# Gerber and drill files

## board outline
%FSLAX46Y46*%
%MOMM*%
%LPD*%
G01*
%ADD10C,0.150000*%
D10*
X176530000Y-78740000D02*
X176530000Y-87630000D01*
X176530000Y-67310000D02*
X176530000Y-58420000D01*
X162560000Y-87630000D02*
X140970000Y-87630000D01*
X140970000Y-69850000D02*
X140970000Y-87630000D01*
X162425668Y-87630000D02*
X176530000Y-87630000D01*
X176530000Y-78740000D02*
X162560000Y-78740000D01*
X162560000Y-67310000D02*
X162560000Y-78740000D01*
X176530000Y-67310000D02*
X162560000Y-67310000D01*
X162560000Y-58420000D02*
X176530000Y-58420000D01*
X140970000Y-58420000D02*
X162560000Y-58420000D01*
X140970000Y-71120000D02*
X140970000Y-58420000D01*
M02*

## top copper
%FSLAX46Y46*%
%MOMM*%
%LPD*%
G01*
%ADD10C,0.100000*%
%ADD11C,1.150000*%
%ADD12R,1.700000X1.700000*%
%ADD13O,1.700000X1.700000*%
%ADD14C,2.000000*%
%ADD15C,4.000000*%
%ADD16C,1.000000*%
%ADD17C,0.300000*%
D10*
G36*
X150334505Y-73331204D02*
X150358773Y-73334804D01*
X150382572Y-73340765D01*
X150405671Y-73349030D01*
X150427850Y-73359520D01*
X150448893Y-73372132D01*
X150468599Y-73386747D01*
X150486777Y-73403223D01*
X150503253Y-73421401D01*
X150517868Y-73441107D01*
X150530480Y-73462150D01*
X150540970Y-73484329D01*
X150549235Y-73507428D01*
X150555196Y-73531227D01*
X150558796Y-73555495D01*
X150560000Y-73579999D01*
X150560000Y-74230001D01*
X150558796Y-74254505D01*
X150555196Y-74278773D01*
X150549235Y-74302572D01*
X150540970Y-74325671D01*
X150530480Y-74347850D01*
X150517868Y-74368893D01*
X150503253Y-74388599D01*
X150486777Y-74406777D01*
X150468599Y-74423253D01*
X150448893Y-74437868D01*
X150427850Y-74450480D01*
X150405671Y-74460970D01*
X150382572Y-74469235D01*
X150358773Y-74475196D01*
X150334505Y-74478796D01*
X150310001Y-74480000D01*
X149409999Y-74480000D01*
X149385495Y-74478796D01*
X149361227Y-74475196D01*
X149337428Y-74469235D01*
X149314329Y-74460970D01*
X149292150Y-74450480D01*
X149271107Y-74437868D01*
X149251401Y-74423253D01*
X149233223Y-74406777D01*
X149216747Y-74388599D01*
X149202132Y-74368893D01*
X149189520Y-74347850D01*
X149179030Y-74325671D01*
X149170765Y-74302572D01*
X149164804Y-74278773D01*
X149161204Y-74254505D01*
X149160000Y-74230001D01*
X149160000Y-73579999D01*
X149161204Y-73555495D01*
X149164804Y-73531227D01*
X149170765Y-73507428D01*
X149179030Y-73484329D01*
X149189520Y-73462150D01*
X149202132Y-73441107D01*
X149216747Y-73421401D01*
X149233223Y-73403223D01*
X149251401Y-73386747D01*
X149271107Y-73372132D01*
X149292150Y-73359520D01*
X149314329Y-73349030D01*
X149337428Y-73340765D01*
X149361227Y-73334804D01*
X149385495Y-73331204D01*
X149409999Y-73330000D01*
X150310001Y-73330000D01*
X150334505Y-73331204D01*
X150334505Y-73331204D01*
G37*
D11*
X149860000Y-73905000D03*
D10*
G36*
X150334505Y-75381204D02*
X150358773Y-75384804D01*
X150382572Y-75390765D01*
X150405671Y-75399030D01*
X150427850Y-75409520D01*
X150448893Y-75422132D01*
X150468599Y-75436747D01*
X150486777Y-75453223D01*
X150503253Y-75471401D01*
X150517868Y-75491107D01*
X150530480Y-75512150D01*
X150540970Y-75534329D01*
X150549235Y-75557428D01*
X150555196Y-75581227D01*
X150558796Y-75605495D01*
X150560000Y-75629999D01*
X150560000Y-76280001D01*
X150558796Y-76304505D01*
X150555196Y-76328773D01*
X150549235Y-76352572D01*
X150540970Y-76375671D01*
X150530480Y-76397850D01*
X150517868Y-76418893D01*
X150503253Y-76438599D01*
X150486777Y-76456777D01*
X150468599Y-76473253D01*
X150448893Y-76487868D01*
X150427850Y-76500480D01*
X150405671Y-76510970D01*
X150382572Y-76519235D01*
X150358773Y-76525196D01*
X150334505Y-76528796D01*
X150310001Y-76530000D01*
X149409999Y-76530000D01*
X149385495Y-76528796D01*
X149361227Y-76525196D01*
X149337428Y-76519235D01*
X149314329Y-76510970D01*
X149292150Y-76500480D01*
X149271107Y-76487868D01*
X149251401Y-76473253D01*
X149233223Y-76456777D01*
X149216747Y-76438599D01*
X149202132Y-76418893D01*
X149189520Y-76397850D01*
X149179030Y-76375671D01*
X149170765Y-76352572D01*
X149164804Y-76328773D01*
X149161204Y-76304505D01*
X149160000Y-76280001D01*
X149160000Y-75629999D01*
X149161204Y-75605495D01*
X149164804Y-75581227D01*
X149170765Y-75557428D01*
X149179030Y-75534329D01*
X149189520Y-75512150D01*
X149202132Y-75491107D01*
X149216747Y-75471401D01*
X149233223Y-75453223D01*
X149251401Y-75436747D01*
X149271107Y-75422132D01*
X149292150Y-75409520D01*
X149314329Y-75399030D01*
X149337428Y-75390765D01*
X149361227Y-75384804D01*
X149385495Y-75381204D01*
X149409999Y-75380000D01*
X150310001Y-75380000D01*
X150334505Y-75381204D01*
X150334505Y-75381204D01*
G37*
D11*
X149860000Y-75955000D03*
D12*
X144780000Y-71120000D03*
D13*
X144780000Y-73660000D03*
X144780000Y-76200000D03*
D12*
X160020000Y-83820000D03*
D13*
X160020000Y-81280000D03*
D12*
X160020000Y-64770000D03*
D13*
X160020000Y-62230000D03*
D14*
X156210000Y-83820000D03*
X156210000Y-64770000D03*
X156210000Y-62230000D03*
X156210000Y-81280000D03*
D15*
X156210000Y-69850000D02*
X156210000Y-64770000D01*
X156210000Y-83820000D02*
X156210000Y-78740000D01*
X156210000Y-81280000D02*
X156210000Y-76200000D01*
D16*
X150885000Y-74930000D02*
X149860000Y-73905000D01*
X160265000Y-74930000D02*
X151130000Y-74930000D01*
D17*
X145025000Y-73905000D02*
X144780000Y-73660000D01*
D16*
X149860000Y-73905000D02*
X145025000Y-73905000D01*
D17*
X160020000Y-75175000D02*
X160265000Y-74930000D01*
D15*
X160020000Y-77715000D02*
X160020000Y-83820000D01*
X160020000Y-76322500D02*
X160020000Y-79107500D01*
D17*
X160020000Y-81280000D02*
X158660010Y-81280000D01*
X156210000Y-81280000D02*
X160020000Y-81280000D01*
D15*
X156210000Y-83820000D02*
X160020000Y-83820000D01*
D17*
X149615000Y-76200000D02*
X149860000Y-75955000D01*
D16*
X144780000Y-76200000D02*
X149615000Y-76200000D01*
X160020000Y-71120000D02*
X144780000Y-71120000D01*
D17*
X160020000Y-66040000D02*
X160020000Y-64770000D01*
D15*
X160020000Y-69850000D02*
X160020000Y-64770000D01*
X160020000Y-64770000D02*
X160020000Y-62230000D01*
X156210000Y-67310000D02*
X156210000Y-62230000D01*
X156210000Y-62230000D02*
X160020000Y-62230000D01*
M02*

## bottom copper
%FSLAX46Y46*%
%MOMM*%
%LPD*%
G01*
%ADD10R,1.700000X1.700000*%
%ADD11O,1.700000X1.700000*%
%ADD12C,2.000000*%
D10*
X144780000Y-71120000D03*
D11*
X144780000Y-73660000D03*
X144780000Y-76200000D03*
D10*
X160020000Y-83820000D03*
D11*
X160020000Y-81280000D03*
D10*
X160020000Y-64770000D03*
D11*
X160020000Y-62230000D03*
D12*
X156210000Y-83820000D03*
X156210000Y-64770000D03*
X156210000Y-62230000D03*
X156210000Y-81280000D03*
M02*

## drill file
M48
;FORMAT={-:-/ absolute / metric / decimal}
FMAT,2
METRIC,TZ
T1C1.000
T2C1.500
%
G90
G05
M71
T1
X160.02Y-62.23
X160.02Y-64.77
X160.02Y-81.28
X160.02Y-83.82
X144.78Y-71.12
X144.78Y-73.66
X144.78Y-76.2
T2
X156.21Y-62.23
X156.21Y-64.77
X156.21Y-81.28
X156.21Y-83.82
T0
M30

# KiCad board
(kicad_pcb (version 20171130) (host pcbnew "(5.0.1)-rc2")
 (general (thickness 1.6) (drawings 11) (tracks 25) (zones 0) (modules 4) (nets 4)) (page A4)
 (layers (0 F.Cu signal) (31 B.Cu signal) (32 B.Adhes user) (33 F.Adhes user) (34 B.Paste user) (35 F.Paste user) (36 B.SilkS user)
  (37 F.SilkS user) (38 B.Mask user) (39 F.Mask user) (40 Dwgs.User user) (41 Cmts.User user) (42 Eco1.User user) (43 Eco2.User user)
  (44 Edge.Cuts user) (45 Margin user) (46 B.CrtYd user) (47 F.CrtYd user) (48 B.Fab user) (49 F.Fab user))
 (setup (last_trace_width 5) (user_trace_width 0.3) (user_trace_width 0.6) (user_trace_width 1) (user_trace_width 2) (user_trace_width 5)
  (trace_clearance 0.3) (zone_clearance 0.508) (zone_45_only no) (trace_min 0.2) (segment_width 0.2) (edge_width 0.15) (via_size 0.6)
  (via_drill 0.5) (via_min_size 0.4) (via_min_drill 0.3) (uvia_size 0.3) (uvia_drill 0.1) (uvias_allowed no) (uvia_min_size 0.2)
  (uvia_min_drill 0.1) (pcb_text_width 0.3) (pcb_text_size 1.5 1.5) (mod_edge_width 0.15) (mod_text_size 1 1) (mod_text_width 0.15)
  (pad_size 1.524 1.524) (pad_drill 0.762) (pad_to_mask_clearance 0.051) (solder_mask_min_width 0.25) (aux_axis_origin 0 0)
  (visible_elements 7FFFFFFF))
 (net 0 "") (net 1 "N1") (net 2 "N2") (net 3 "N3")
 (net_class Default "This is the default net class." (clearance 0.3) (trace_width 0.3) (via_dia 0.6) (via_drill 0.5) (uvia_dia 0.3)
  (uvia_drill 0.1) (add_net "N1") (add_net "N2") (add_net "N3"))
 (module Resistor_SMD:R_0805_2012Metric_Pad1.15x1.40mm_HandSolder (layer F.Cu) (at 149.86 74.93 270)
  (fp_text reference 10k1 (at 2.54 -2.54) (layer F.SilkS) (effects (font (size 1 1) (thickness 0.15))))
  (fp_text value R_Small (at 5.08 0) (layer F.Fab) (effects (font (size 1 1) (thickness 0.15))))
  (pad 1 smd roundrect (at -1.025 0 270) (size 1.15 1.4) (layers F.Cu F.Paste F.Mask) (roundrect_rratio 0.217391) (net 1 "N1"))
  (pad 2 smd roundrect (at 1.025 0 270) (size 1.15 1.4) (layers F.Cu F.Paste F.Mask) (roundrect_rratio 0.217391) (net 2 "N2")))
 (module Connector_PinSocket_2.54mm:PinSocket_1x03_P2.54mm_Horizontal (layer F.Cu) (at 144.78 71.12)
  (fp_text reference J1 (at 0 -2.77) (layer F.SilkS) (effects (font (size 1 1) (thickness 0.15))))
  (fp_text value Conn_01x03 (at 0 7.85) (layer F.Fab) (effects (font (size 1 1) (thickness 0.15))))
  (pad 1 thru_hole rect (at 0 0) (size 1.7 1.7) (drill 1) (layers *.Cu *.Mask) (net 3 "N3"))
  (pad 2 thru_hole oval (at 0 2.54) (size 1.7 1.7) (drill 1) (layers *.Cu *.Mask) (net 1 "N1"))
  (pad 3 thru_hole oval (at 0 5.08) (size 1.7 1.7) (drill 1) (layers *.Cu *.Mask) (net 2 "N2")))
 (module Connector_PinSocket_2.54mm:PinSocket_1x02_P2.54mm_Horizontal (layer F.Cu) (at 160.02 83.82 180)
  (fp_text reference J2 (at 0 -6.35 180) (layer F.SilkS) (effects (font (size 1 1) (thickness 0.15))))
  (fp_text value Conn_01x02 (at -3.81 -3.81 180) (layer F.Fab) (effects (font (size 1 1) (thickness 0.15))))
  (pad 1 thru_hole rect (at 0 0 180) (size 1.7 1.7) (drill 1) (layers *.Cu *.Mask) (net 1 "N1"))
  (pad 2 thru_hole oval (at 0 2.54 180) (size 1.7 1.7) (drill 1) (layers *.Cu *.Mask) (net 1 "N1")))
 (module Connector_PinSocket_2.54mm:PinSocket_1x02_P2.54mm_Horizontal (layer F.Cu) (at 160.02 64.77 180)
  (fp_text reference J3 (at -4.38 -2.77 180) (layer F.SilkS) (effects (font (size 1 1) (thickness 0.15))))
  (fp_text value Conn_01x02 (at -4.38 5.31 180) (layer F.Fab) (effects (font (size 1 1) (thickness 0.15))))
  (pad 1 thru_hole rect (at 0 0 180) (size 1.7 1.7) (drill 1) (layers *.Cu *.Mask) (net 3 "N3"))
  (pad 2 thru_hole oval (at 0 2.54 180) (size 1.7 1.7) (drill 1) (layers *.Cu *.Mask) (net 3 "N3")))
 (gr_line (start 176.53 78.74) (end 176.53 87.63) (layer Edge.Cuts) (width 0.15))
 (gr_line (start 176.53 67.31) (end 176.53 58.42) (layer Edge.Cuts) (width 0.15))
 (gr_line (start 162.56 87.63) (end 140.97 87.63) (layer Edge.Cuts) (width 0.15))
 (gr_line (start 140.97 69.85) (end 140.97 87.63) (layer Edge.Cuts) (width 0.15))
 (gr_line (start 162.425668 87.63) (end 176.53 87.63) (layer Edge.Cuts) (width 0.15))
 (gr_line (start 176.53 78.74) (end 162.56 78.74) (layer Edge.Cuts) (width 0.15))
 (gr_line (start 162.56 67.31) (end 162.56 78.74) (layer Edge.Cuts) (width 0.15))
 (gr_line (start 176.53 67.31) (end 162.56 67.31) (layer Edge.Cuts) (width 0.15))
 (gr_line (start 162.56 58.42) (end 176.53 58.42) (layer Edge.Cuts) (width 0.15))
 (gr_line (start 140.97 58.42) (end 162.56 58.42) (layer Edge.Cuts) (width 0.15))
 (gr_line (start 140.97 71.12) (end 140.97 58.42) (layer Edge.Cuts) (width 0.15))
 (via (at 156.21 83.82) (size 2) (drill 1.5) (layers F.Cu B.Cu) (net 1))
 (via (at 156.21 64.77) (size 2) (drill 1.5) (layers F.Cu B.Cu) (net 3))
 (via (at 156.21 62.23) (size 2) (drill 1.5) (layers F.Cu B.Cu) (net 3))
 (segment (start 156.21 69.85) (end 156.21 64.77) (width 4) (layer F.Cu) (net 3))
 (segment (start 156.21 83.82) (end 156.21 78.74) (width 4) (layer F.Cu) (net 1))
 (segment (start 156.21 81.28) (end 156.21 76.2) (width 4) (layer F.Cu) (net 1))
 (via (at 156.21 81.28) (size 2) (drill 1.5) (layers F.Cu B.Cu) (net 1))
 (segment (start 150.885 74.93) (end 149.86 73.905) (width 1) (layer F.Cu) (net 1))
 (segment (start 160.265 74.93) (end 151.13 74.93) (width 1) (layer F.Cu) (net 1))
 (segment (start 145.025 73.905) (end 144.78 73.66) (width 0.3) (layer F.Cu) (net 1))
 (segment (start 149.86 73.905) (end 145.025 73.905) (width 1) (layer F.Cu) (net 1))
 (segment (start 160.02 75.175) (end 160.265 74.93) (width 0.3) (layer F.Cu) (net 1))
 (segment (start 160.02 77.715) (end 160.02 83.82) (width 4) (layer F.Cu) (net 1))
 (segment (start 160.02 76.3225) (end 160.02 79.1075) (width 4) (layer F.Cu) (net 1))
 (segment (start 160.02 81.28) (end 158.66001 81.28) (width 0.3) (layer F.Cu) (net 1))
 (segment (start 156.21 81.28) (end 160.02 81.28) (width 0.3) (layer F.Cu) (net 1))
 (segment (start 156.21 83.82) (end 160.02 83.82) (width 4) (layer F.Cu) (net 1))
 (segment (start 149.615 76.2) (end 149.86 75.955) (width 0.3) (layer F.Cu) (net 2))
 (segment (start 144.78 76.2) (end 149.615 76.2) (width 1) (layer F.Cu) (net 2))
 (segment (start 160.02 71.12) (end 144.78 71.12) (width 1) (layer F.Cu) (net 3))
 (segment (start 160.02 66.04) (end 160.02 64.77) (width 0.3) (layer F.Cu) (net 3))
 (segment (start 160.02 69.85) (end 160.02 64.77) (width 4) (layer F.Cu) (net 3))
 (segment (start 160.02 64.77) (end 160.02 62.23) (width 4) (layer F.Cu) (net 3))
 (segment (start 156.21 67.31) (end 156.21 62.23) (width 4) (layer F.Cu) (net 3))
 (segment (start 156.21 62.23) (end 160.02 62.23) (width 4) (layer F.Cu) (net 3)))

